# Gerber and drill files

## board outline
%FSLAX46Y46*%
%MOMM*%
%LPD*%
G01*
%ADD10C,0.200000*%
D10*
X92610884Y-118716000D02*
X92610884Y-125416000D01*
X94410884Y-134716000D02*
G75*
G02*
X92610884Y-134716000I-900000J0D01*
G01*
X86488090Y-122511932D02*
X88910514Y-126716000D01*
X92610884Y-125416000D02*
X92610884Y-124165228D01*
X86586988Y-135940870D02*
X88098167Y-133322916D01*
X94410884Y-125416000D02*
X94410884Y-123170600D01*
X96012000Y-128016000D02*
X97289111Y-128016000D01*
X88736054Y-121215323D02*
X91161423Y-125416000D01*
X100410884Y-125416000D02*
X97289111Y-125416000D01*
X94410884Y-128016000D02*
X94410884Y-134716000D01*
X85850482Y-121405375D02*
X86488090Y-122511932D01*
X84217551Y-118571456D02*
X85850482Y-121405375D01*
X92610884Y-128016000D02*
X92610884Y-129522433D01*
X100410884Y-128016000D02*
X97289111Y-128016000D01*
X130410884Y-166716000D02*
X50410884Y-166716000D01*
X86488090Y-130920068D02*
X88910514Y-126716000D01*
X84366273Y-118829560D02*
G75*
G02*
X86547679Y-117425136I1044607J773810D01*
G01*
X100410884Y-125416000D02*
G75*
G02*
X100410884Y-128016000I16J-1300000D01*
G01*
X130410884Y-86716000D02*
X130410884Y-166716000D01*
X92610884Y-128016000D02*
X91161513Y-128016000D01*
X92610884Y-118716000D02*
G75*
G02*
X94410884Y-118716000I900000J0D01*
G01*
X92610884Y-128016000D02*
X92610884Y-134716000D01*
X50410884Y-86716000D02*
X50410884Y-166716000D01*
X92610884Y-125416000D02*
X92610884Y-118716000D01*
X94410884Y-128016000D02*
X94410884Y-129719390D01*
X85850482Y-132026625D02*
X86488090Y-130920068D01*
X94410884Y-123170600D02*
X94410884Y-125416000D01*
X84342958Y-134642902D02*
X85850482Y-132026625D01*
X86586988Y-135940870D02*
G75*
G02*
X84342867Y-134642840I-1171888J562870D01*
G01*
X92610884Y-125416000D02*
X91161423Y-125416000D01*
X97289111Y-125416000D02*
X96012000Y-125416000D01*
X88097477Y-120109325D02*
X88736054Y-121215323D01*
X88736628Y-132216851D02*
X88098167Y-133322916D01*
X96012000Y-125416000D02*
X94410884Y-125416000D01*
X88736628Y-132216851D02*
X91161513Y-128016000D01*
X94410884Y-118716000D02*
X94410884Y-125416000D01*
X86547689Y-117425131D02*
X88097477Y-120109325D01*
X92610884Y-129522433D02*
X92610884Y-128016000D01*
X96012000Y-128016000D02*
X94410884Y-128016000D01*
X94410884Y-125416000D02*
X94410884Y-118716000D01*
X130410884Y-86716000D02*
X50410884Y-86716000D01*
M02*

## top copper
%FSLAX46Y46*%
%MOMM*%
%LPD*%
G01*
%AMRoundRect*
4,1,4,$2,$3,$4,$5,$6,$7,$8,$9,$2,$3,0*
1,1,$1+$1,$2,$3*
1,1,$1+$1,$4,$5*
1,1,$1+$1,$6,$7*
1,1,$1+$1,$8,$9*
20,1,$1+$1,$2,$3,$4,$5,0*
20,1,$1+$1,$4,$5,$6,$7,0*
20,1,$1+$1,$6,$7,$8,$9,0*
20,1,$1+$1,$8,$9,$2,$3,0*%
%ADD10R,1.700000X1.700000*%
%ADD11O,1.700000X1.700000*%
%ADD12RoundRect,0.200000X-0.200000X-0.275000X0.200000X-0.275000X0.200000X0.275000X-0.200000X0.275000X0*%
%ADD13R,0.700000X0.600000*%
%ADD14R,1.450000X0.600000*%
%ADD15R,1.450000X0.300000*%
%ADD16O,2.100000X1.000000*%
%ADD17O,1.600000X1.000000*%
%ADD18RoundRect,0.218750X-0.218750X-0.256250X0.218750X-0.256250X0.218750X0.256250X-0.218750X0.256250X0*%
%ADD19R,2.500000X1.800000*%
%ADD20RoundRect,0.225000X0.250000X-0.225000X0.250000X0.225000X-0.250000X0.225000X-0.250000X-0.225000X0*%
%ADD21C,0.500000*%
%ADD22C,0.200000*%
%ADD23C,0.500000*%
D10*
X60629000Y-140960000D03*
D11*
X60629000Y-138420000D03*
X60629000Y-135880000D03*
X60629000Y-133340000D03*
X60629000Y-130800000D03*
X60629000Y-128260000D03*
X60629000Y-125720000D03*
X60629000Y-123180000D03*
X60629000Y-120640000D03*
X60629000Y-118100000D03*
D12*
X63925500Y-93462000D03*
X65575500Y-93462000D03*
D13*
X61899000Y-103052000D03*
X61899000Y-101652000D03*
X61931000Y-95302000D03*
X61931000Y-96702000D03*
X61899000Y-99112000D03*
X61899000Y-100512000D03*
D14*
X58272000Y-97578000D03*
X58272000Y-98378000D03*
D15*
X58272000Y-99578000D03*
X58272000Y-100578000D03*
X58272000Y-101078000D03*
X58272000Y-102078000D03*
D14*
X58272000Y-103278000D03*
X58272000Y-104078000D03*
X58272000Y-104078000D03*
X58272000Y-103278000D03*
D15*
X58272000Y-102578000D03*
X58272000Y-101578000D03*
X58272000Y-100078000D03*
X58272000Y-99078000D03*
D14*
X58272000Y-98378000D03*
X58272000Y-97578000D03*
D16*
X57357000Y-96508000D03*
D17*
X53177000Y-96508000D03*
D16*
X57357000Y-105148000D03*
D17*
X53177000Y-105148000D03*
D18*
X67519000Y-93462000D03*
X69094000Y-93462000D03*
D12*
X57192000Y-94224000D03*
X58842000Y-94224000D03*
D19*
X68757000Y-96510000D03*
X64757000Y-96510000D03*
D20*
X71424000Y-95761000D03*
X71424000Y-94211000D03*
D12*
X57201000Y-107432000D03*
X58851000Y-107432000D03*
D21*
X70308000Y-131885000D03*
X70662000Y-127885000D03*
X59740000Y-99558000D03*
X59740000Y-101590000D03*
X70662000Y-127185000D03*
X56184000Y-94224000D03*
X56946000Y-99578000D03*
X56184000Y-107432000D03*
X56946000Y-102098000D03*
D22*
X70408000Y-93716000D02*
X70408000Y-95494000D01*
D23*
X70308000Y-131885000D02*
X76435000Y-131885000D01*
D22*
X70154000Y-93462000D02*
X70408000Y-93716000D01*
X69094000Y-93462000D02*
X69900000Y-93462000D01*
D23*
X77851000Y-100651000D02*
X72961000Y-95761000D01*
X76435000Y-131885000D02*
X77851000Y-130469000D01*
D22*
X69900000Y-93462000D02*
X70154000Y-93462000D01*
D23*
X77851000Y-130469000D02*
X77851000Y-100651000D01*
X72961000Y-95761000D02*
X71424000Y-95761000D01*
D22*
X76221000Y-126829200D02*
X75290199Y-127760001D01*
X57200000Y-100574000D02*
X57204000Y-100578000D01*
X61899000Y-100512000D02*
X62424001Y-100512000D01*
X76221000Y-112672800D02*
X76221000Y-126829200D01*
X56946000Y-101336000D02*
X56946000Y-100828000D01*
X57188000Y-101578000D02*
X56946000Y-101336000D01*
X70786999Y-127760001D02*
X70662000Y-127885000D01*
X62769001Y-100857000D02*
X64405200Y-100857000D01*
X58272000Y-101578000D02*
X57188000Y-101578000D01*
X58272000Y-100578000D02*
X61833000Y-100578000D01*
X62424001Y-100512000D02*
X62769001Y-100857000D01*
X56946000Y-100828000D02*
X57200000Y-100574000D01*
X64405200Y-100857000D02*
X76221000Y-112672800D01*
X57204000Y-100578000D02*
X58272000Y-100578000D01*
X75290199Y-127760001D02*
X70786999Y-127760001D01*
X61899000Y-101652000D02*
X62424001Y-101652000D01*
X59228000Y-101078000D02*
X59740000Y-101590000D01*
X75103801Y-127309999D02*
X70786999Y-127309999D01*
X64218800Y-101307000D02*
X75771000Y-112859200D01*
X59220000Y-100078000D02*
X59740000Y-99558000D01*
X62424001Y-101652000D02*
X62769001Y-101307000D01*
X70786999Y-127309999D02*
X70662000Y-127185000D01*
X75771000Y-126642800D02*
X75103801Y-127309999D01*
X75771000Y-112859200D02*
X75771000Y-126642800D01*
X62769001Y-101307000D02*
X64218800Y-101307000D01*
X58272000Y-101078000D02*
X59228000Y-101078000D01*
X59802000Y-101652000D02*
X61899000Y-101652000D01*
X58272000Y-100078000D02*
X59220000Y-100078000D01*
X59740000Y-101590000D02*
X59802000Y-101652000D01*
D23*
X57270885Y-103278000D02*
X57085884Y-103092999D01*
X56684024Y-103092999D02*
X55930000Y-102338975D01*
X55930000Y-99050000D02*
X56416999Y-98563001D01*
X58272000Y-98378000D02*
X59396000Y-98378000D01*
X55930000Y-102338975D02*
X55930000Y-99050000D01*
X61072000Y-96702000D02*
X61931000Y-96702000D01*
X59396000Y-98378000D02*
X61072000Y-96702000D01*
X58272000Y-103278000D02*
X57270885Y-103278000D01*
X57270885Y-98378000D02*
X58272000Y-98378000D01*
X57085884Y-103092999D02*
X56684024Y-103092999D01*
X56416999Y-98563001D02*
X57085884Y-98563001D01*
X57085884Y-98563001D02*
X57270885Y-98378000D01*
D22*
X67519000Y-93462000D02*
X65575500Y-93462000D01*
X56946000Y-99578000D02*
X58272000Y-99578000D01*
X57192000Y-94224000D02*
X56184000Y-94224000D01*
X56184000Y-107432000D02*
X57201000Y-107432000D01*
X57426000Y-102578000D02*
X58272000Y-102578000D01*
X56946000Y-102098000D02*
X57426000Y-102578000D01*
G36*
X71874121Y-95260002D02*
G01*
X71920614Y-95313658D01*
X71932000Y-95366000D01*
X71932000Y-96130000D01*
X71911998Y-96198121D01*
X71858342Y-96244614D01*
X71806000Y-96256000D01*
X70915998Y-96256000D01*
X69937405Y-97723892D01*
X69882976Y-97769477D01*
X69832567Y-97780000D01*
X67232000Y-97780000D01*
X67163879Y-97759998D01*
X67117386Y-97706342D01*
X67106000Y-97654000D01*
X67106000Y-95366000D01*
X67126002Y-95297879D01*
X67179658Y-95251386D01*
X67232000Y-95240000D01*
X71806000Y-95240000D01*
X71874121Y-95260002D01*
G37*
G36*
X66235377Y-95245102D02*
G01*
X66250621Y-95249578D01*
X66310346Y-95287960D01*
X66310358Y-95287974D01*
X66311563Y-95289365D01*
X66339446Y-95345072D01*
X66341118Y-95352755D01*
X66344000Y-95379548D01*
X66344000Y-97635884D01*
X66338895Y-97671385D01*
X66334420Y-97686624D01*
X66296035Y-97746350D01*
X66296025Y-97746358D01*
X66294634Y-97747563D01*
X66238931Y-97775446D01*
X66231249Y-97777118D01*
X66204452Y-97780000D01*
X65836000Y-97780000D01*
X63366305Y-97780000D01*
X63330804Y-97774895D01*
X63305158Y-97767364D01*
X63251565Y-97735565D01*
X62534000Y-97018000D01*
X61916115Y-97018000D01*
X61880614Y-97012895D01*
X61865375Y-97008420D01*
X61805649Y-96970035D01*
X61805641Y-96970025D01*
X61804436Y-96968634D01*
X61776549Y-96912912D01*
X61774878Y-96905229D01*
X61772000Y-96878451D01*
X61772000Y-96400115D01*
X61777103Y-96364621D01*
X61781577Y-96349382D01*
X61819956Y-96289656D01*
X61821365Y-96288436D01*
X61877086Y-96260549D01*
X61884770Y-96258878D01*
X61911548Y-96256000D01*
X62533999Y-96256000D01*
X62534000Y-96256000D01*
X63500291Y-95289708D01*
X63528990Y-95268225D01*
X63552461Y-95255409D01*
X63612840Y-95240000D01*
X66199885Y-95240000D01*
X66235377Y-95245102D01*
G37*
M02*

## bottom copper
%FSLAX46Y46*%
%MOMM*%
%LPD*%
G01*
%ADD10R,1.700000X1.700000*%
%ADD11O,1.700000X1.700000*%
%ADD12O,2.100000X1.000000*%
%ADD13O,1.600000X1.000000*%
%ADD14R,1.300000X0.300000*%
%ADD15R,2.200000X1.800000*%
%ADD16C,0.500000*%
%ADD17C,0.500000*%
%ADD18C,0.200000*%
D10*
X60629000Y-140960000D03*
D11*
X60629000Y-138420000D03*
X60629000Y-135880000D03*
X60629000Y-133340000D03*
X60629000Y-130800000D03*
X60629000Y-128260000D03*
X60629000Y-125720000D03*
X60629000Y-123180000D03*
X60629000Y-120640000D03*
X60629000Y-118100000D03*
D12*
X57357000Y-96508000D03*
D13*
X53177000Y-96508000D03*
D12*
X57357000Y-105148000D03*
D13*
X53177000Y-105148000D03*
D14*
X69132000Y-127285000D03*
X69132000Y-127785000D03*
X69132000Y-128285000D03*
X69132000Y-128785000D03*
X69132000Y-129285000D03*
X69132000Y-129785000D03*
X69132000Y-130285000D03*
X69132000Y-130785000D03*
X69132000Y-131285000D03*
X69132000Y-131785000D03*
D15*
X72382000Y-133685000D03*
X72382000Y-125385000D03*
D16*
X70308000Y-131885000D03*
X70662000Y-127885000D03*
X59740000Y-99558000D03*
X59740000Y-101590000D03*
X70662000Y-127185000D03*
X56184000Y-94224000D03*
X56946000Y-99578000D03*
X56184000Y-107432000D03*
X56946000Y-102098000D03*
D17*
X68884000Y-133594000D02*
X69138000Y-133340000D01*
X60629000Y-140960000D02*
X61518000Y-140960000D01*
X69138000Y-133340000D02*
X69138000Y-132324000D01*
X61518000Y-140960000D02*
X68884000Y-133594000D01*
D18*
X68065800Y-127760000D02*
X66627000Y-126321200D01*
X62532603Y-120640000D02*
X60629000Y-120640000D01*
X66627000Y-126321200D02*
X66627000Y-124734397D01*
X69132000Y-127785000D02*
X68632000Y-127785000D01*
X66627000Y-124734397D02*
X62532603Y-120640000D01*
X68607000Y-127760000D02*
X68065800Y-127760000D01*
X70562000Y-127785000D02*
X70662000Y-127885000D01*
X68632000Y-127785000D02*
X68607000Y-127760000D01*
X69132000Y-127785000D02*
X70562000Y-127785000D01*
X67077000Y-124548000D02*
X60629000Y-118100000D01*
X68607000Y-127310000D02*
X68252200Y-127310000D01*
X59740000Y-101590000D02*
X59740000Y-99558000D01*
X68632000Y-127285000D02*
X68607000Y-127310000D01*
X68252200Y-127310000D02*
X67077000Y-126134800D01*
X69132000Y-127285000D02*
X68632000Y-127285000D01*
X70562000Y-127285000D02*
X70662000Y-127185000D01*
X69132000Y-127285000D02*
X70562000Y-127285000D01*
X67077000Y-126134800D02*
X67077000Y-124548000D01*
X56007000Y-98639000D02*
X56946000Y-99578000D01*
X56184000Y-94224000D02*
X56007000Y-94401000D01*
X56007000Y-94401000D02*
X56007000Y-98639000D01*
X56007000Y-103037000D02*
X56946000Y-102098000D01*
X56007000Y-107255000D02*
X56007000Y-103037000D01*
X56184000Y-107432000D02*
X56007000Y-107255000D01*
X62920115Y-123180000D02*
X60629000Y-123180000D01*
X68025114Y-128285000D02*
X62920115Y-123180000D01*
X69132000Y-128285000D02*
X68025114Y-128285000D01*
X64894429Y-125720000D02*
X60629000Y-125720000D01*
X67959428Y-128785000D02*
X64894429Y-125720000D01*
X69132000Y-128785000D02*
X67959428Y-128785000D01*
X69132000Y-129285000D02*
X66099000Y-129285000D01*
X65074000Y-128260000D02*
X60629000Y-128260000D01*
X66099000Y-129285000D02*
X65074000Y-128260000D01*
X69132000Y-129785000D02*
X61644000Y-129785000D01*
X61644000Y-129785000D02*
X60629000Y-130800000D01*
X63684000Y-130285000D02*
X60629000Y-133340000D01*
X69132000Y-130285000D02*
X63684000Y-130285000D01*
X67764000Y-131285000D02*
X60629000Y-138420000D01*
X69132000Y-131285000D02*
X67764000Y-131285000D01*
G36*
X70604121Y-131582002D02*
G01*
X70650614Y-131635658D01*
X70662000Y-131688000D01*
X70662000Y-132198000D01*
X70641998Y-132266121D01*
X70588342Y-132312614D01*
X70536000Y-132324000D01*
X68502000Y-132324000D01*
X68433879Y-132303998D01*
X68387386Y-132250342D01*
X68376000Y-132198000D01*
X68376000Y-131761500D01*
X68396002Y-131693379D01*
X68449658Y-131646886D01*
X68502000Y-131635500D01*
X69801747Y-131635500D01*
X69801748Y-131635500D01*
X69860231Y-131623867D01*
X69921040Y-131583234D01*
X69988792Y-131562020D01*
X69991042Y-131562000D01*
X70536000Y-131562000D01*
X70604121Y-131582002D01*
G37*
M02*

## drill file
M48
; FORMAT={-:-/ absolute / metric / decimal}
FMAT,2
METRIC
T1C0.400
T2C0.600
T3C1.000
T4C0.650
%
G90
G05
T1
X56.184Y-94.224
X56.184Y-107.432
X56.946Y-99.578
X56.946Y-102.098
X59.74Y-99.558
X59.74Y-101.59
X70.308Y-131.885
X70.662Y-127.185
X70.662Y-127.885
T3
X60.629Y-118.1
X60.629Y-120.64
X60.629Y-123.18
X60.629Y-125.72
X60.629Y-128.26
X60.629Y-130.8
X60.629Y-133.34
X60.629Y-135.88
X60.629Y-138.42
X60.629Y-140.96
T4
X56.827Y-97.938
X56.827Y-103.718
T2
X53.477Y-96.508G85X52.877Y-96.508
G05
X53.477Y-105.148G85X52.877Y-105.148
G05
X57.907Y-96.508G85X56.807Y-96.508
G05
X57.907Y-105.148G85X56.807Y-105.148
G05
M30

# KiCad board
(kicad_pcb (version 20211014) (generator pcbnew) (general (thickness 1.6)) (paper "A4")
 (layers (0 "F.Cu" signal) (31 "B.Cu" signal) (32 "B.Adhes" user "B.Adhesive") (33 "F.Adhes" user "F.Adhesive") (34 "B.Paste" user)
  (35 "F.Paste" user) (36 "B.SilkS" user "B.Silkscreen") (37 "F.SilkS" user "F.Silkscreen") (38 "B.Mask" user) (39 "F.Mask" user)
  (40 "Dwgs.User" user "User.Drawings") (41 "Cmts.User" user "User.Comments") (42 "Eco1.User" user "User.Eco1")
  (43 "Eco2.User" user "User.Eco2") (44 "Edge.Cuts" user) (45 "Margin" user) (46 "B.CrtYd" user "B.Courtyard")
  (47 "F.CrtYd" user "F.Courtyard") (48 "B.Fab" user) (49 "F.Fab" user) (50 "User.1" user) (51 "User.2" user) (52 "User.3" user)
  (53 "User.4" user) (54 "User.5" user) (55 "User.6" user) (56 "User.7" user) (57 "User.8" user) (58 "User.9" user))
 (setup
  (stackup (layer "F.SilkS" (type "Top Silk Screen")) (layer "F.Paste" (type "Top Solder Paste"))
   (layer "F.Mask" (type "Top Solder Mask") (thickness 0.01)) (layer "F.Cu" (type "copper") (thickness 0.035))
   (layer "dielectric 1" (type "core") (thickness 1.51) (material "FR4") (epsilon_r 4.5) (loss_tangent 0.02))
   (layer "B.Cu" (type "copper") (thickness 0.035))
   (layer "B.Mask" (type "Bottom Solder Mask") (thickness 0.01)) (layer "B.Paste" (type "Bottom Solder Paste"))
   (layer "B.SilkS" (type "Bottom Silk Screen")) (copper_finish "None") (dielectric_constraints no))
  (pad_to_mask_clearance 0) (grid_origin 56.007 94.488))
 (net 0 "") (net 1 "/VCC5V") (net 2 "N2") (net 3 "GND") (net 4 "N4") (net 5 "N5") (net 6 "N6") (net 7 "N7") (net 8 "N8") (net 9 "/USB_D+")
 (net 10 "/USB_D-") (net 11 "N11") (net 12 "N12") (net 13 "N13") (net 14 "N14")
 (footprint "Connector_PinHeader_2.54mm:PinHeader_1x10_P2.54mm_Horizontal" (layer "F.Cu") (at 60.629 140.96 180)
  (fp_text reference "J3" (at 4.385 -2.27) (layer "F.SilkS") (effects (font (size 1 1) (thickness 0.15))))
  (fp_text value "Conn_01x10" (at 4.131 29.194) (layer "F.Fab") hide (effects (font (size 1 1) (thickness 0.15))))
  (pad "1" thru_hole rect (at 0 0 180) (size 1.7 1.7) (drill 1) (layers *.Cu *.Mask) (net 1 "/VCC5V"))
  (pad "2" thru_hole oval (at 0 2.54 180) (size 1.7 1.7) (drill 1) (layers *.Cu *.Mask) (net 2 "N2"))
  (pad "3" thru_hole oval (at 0 5.08 180) (size 1.7 1.7) (drill 1) (layers *.Cu *.Mask) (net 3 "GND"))
  (pad "4" thru_hole oval (at 0 7.62 180) (size 1.7 1.7) (drill 1) (layers *.Cu *.Mask) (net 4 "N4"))
  (pad "5" thru_hole oval (at 0 10.16 180) (size 1.7 1.7) (drill 1) (layers *.Cu *.Mask) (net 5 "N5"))
  (pad "6" thru_hole oval (at 0 12.7 180) (size 1.7 1.7) (drill 1) (layers *.Cu *.Mask) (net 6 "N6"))
  (pad "7" thru_hole oval (at 0 15.24 180) (size 1.7 1.7) (drill 1) (layers *.Cu *.Mask) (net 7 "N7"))
  (pad "8" thru_hole oval (at 0 17.78 180) (size 1.7 1.7) (drill 1) (layers *.Cu *.Mask) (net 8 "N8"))
  (pad "9" thru_hole oval (at 0 20.32 180) (size 1.7 1.7) (drill 1) (layers *.Cu *.Mask) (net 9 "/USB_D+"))
  (pad "10" thru_hole oval (at 0 22.86 180) (size 1.7 1.7) (drill 1) (layers *.Cu *.Mask) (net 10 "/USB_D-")))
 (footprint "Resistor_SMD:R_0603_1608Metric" (layer "F.Cu") (at 64.7505 93.462)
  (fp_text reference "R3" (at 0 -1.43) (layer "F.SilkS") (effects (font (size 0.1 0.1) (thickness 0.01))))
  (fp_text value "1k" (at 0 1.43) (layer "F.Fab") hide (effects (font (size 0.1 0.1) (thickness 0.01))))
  (pad "1" smd roundrect (at -0.825 0) (size 0.8 0.95) (layers "F.Cu" "F.Paste" "F.Mask") (roundrect_rratio 0.25) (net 3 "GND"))
  (pad "2" smd roundrect (at 0.825 0) (size 0.8 0.95) (layers "F.Cu" "F.Paste" "F.Mask") (roundrect_rratio 0.25) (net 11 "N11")))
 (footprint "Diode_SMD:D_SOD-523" (layer "F.Cu") (at 61.899 102.352 90)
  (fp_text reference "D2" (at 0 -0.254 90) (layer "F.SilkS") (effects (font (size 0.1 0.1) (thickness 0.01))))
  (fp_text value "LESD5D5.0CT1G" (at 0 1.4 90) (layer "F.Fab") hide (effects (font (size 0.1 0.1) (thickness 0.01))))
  (pad "1" smd rect (at -0.7 0 270) (size 0.6 0.7) (layers "F.Cu" "F.Paste" "F.Mask") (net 3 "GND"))
  (pad "2" smd rect (at 0.7 0 270) (size 0.6 0.7) (layers "F.Cu" "F.Paste" "F.Mask") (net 10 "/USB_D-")))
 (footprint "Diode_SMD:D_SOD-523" (layer "F.Cu") (at 61.931 96.002 -90)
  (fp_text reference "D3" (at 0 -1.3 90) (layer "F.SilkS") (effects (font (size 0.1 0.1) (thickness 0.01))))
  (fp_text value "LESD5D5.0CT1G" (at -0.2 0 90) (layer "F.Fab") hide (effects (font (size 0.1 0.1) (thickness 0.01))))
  (pad "1" smd rect (at -0.7 0 90) (size 0.6 0.7) (layers "F.Cu" "F.Paste" "F.Mask") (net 3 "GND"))
  (pad "2" smd rect (at 0.7 0 90) (size 0.6 0.7) (layers "F.Cu" "F.Paste" "F.Mask") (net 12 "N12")))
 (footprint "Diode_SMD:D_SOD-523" (layer "F.Cu") (at 61.899 99.812 -90)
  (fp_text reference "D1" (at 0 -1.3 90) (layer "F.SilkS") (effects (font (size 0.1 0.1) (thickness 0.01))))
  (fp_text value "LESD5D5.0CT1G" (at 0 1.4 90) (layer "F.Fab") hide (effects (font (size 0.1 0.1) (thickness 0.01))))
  (pad "1" smd rect (at -0.7 0 90) (size 0.6 0.7) (layers "F.Cu" "F.Paste" "F.Mask") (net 3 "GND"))
  (pad "2" smd rect (at 0.7 0 90) (size 0.6 0.7) (layers "F.Cu" "F.Paste" "F.Mask") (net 9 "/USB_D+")))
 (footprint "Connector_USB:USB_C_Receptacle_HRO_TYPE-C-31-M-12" (layer "F.Cu") (at 54.227 100.828 -90)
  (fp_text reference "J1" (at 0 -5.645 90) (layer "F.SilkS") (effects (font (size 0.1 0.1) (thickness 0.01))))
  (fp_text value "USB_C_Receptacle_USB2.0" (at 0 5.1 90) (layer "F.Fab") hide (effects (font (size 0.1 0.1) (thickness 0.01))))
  (pad "" np_thru_hole circle (at 2.89 -2.6 270) (size 0.65 0.65) (drill 0.65) (layers *.Cu *.Mask))
  (pad "" np_thru_hole circle (at -2.89 -2.6 270) (size 0.65 0.65) (drill 0.65) (layers *.Cu *.Mask))
  (pad "A1" smd rect (at -3.25 -4.045 270) (size 0.6 1.45) (layers "F.Cu" "F.Paste" "F.Mask") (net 3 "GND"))
  (pad "A4" smd rect (at -2.45 -4.045 270) (size 0.6 1.45) (layers "F.Cu" "F.Paste" "F.Mask") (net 12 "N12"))
  (pad "A5" smd rect (at -1.25 -4.045 270) (size 0.3 1.45) (layers "F.Cu" "F.Paste" "F.Mask") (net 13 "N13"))
  (pad "A6" smd rect locked (at -0.25 -4.045 270) (size 0.3 1.45) (layers "F.Cu" "F.Paste" "F.Mask") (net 9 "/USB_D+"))
  (pad "A7" smd rect (at 0.25 -4.045 270) (size 0.3 1.45) (layers "F.Cu" "F.Paste" "F.Mask") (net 10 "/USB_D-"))
  (pad "A8" smd rect (at 1.25 -4.045 270) (size 0.3 1.45) (layers "F.Cu" "F.Paste" "F.Mask") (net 3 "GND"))
  (pad "A9" smd rect (at 2.45 -4.045 270) (size 0.6 1.45) (layers "F.Cu" "F.Paste" "F.Mask") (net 12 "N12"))
  (pad "A12" smd rect (at 3.25 -4.045 270) (size 0.6 1.45) (layers "F.Cu" "F.Paste" "F.Mask") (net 3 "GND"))
  (pad "B1" smd rect (at 3.25 -4.045 270) (size 0.6 1.45) (layers "F.Cu" "F.Paste" "F.Mask") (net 3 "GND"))
  (pad "B4" smd rect (at 2.45 -4.045 270) (size 0.6 1.45) (layers "F.Cu" "F.Paste" "F.Mask") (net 12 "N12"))
  (pad "B5" smd rect (at 1.75 -4.045 270) (size 0.3 1.45) (layers "F.Cu" "F.Paste" "F.Mask") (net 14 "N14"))
  (pad "B6" smd rect (at 0.75 -4.045 270) (size 0.3 1.45) (layers "F.Cu" "F.Paste" "F.Mask") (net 9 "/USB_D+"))
  (pad "B7" smd rect (at -0.75 -4.045 270) (size 0.3 1.45) (layers "F.Cu" "F.Paste" "F.Mask") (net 10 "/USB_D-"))
  (pad "B8" smd rect (at -1.75 -4.045 270) (size 0.3 1.45) (layers "F.Cu" "F.Paste" "F.Mask") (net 3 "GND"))
  (pad "B9" smd rect (at -2.45 -4.045 270) (size 0.6 1.45) (layers "F.Cu" "F.Paste" "F.Mask") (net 12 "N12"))
  (pad "B12" smd rect (at -3.25 -4.045 270) (size 0.6 1.45) (layers "F.Cu" "F.Paste" "F.Mask") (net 3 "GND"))
  (pad "S1" thru_hole oval (at -4.32 -3.13 270) (size 1 2.1) (drill oval 0.6 1.7) (layers *.Cu *.Mask) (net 3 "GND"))
  (pad "S1" thru_hole oval (at -4.32 1.05 270) (size 1 1.6) (drill oval 0.6 1.2) (layers *.Cu *.Mask) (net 3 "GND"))
  (pad "S1" thru_hole oval (at 4.32 -3.13 270) (size 1 2.1) (drill oval 0.6 1.7) (layers *.Cu *.Mask) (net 3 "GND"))
  (pad "S1" thru_hole oval (at 4.32 1.05 270) (size 1 1.6) (drill oval 0.6 1.2) (layers *.Cu *.Mask) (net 3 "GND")))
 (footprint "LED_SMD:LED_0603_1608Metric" (layer "F.Cu") (at 68.3065 93.462)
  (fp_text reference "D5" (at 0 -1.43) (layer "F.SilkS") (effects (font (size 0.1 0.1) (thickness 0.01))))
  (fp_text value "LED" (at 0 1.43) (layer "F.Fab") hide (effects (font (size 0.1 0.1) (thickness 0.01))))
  (pad "1" smd roundrect (at -0.7875 0) (size 0.875 0.95) (layers "F.Cu" "F.Paste" "F.Mask") (roundrect_rratio 0.25) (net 11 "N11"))
  (pad "2" smd roundrect (at 0.7875 0) (size 0.875 0.95) (layers "F.Cu" "F.Paste" "F.Mask") (roundrect_rratio 0.25) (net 1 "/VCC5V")))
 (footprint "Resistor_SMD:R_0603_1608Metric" (layer "F.Cu") (at 58.017 94.224)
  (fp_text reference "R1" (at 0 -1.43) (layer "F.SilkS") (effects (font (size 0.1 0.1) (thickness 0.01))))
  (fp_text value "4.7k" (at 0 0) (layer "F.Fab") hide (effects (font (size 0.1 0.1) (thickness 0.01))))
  (pad "1" smd roundrect (at -0.825 0) (size 0.8 0.95) (layers "F.Cu" "F.Paste" "F.Mask") (roundrect_rratio 0.25) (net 13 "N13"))
  (pad "2" smd roundrect (at 0.825 0) (size 0.8 0.95) (layers "F.Cu" "F.Paste" "F.Mask") (roundrect_rratio 0.25) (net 3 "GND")))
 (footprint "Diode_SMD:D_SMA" (layer "F.Cu") (at 66.757 96.51 180)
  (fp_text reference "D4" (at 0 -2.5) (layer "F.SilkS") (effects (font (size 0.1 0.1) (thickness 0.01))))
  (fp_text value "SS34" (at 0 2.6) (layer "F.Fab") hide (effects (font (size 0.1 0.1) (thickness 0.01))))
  (pad "1" smd rect (at -2 0 180) (size 2.5 1.8) (layers "F.Cu" "F.Paste" "F.Mask") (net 1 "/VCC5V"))
  (pad "2" smd rect (at 2 0 180) (size 2.5 1.8) (layers "F.Cu" "F.Paste" "F.Mask") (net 12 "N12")))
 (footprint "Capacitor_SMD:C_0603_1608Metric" (layer "F.Cu") (at 71.424 94.986 90)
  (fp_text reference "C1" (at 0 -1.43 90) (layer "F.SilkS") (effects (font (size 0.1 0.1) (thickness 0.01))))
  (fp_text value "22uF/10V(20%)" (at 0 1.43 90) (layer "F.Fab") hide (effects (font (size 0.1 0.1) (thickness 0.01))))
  (pad "1" smd roundrect (at -0.775 0 90) (size 0.9 0.95) (layers "F.Cu" "F.Paste" "F.Mask") (roundrect_rratio 0.25) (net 1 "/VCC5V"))
  (pad "2" smd roundrect (at 0.775 0 90) (size 0.9 0.95) (layers "F.Cu" "F.Paste" "F.Mask") (roundrect_rratio 0.25) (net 3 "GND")))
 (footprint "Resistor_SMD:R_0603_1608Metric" (layer "F.Cu") (at 58.026 107.432)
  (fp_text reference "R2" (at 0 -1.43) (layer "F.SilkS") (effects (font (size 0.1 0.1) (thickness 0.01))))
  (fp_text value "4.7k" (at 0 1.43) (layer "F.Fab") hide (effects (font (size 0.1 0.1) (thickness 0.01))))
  (pad "1" smd roundrect (at -0.825 0) (size 0.8 0.95) (layers "F.Cu" "F.Paste" "F.Mask") (roundrect_rratio 0.25) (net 14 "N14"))
  (pad "2" smd roundrect (at 0.825 0) (size 0.8 0.95) (layers "F.Cu" "F.Paste" "F.Mask") (roundrect_rratio 0.25) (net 3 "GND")))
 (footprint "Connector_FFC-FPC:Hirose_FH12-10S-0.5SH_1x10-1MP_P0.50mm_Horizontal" (layer "B.Cu") (at 70.982 129.535 -90)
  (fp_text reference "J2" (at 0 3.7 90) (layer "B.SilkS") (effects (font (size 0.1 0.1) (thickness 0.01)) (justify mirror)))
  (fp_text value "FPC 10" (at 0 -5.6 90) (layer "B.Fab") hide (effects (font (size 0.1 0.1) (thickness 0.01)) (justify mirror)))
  (pad "1" smd rect (at -2.25 1.85 270) (size 0.3 1.3) (layers "B.Cu" "B.Paste" "B.Mask") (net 10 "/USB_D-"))
  (pad "2" smd rect (at -1.75 1.85 270) (size 0.3 1.3) (layers "B.Cu" "B.Paste" "B.Mask") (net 9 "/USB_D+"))
  (pad "3" smd rect (at -1.25 1.85 270) (size 0.3 1.3) (layers "B.Cu" "B.Paste" "B.Mask") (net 8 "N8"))
  (pad "4" smd rect (at -0.75 1.85 270) (size 0.3 1.3) (layers "B.Cu" "B.Paste" "B.Mask") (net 7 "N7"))
  (pad "5" smd rect (at -0.25 1.85 270) (size 0.3 1.3) (layers "B.Cu" "B.Paste" "B.Mask") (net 6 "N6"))
  (pad "6" smd rect (at 0.25 1.85 270) (size 0.3 1.3) (layers "B.Cu" "B.Paste" "B.Mask") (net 5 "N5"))
  (pad "7" smd rect (at 0.75 1.85 270) (size 0.3 1.3) (layers "B.Cu" "B.Paste" "B.Mask") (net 4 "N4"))
  (pad "8" smd rect (at 1.25 1.85 270) (size 0.3 1.3) (layers "B.Cu" "B.Paste" "B.Mask") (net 3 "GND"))
  (pad "9" smd rect (at 1.75 1.85 270) (size 0.3 1.3) (layers "B.Cu" "B.Paste" "B.Mask") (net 2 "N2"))
  (pad "10" smd rect (at 2.25 1.85 270) (size 0.3 1.3) (layers "B.Cu" "B.Paste" "B.Mask") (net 1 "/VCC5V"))
  (pad "MP" smd rect (at 4.15 -1.4 270) (size 1.8 2.2) (layers "B.Cu" "B.Paste" "B.Mask"))
  (pad "MP" smd rect (at -4.15 -1.4 270) (size 1.8 2.2) (layers "B.Cu" "B.Paste" "B.Mask")))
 (gr_line (start 92.610884 118.716) (end 92.610884 125.416) (layer "Edge.Cuts") (width 0.2))
 (gr_arc (start 94.410884 134.716) (mid 93.510884 135.616) (end 92.610884 134.716) (layer "Edge.Cuts") (width 0.2))
 (gr_line (start 86.48809 122.511932) (end 88.910514 126.716) (layer "Edge.Cuts") (width 0.2))
 (gr_line (start 92.610884 125.416) (end 92.610884 124.165228) (layer "Edge.Cuts") (width 0.2))
 (gr_line (start 86.586988 135.94087) (end 88.098167 133.322916) (layer "Edge.Cuts") (width 0.2))
 (gr_line (start 94.410884 125.416) (end 94.410884 123.1706) (layer "Edge.Cuts") (width 0.2))
 (gr_line (start 96.012 128.016) (end 97.289111 128.016) (layer "Edge.Cuts") (width 0.2))
 (gr_line (start 88.736054 121.215323) (end 91.161423 125.416) (layer "Edge.Cuts") (width 0.2))
 (gr_line (start 100.410884 125.416) (end 97.289111 125.416) (layer "Edge.Cuts") (width 0.2))
 (gr_line (start 94.410884 128.016) (end 94.410884 134.716) (layer "Edge.Cuts") (width 0.2))
 (gr_line (start 85.850482 121.405375) (end 86.48809 122.511932) (layer "Edge.Cuts") (width 0.2))
 (gr_line (start 84.217551 118.571456) (end 85.850482 121.405375) (layer "Edge.Cuts") (width 0.2))
 (gr_line (start 92.610884 128.016) (end 92.610884 129.522433) (layer "Edge.Cuts") (width 0.2))
 (gr_line (start 100.410884 128.016) (end 97.289111 128.016) (layer "Edge.Cuts") (width 0.2))
 (gr_line (start 130.410884 166.716) (end 50.410884 166.716) (layer "Edge.Cuts") (width 0.2))
 (gr_line (start 86.48809 130.920068) (end 88.910514 126.716) (layer "Edge.Cuts") (width 0.2))
 (gr_arc (start 84.366273 118.82956) (mid 84.707158 116.962691) (end 86.547689 117.425131) (layer "Edge.Cuts") (width 0.2))
 (gr_arc (start 100.410884 125.416) (mid 101.710884 126.716) (end 100.410884 128.016) (layer "Edge.Cuts") (width 0.2))
 (gr_line (start 130.410884 86.716) (end 130.410884 166.716) (layer "Edge.Cuts") (width 0.2))
 (gr_line (start 92.610884 128.016) (end 91.161513 128.016) (layer "Edge.Cuts") (width 0.2))
 (gr_arc (start 92.610884 118.716) (mid 93.510884 117.816) (end 94.410884 118.716) (layer "Edge.Cuts") (width 0.2))
 (gr_line (start 92.610884 128.016) (end 92.610884 134.716) (layer "Edge.Cuts") (width 0.2))
 (gr_line (start 50.410884 86.716) (end 50.410884 166.716) (layer "Edge.Cuts") (width 0.2))
 (gr_line (start 92.610884 125.416) (end 92.610884 118.716) (layer "Edge.Cuts") (width 0.2))
 (gr_line (start 94.410884 128.016) (end 94.410884 129.71939) (layer "Edge.Cuts") (width 0.2))
 (gr_line (start 85.850482 132.026625) (end 86.48809 130.920068) (layer "Edge.Cuts") (width 0.2))
 (gr_line (start 94.410884 123.1706) (end 94.410884 125.416) (layer "Edge.Cuts") (width 0.2))
 (gr_line (start 84.342958 134.642902) (end 85.850482 132.026625) (layer "Edge.Cuts") (width 0.2))
 (gr_arc (start 86.586988 135.94087) (mid 84.764255 136.503343) (end 84.342958 134.642902) (layer "Edge.Cuts") (width 0.2))
 (gr_line (start 92.610884 125.416) (end 91.161423 125.416) (layer "Edge.Cuts") (width 0.2))
 (gr_line (start 97.289111 125.416) (end 96.012 125.416) (layer "Edge.Cuts") (width 0.2))
 (gr_line (start 88.097477 120.109325) (end 88.736054 121.215323) (layer "Edge.Cuts") (width 0.2))
 (gr_line (start 88.736628 132.216851) (end 88.098167 133.322916) (layer "Edge.Cuts") (width 0.2))
 (gr_line (start 96.012 125.416) (end 94.410884 125.416) (layer "Edge.Cuts") (width 0.2))
 (gr_line (start 88.736628 132.216851) (end 91.161513 128.016) (layer "Edge.Cuts") (width 0.2))
 (gr_line (start 94.410884 118.716) (end 94.410884 125.416) (layer "Edge.Cuts") (width 0.2))
 (gr_line (start 86.547689 117.425131) (end 88.097477 120.109325) (layer "Edge.Cuts") (width 0.2))
 (gr_line (start 92.610884 129.522433) (end 92.610884 128.016) (layer "Edge.Cuts") (width 0.2))
 (gr_line (start 96.012 128.016) (end 94.410884 128.016) (layer "Edge.Cuts") (width 0.2))
 (gr_line (start 94.410884 125.416) (end 94.410884 118.716) (layer "Edge.Cuts") (width 0.2))
 (gr_line (start 130.410884 86.716) (end 50.410884 86.716) (layer "Edge.Cuts") (width 0.2))
 (segment (start 70.408 93.716) (end 70.408 95.494) (width 0.2) (layer "F.Cu") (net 1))
 (segment (start 70.308 131.885) (end 76.435 131.885) (width 0.5) (layer "F.Cu") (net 1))
 (segment (start 70.154 93.462) (end 70.408 93.716) (width 0.2) (layer "F.Cu") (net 1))
 (segment (start 69.094 93.462) (end 69.9 93.462) (width 0.2) (layer "F.Cu") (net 1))
 (segment (start 77.851 100.651) (end 72.961 95.761) (width 0.5) (layer "F.Cu") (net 1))
 (segment (start 76.435 131.885) (end 77.851 130.469) (width 0.5) (layer "F.Cu") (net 1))
 (segment (start 69.9 93.462) (end 70.154 93.462) (width 0.2) (layer "F.Cu") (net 1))
 (segment (start 77.851 130.469) (end 77.851 100.651) (width 0.5) (layer "F.Cu") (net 1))
 (segment (start 72.961 95.761) (end 71.424 95.761) (width 0.5) (layer "F.Cu") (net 1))
 (via (at 70.308 131.885) (size 0.5) (drill 0.4) (layers "F.Cu" "B.Cu") (free) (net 1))
 (segment (start 68.884 133.594) (end 69.138 133.34) (width 0.5) (layer "B.Cu") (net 1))
 (segment (start 60.629 140.96) (end 61.518 140.96) (width 0.5) (layer "B.Cu") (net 1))
 (segment (start 69.138 133.34) (end 69.138 132.324) (width 0.5) (layer "B.Cu") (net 1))
 (segment (start 61.518 140.96) (end 68.884 133.594) (width 0.5) (layer "B.Cu") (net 1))
 (segment (start 76.221 126.8292) (end 75.290199 127.760001) (width 0.2) (layer "F.Cu") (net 9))
 (segment (start 57.2 100.574) (end 57.204 100.578) (width 0.2) (layer "F.Cu") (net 9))
 (segment (start 61.899 100.512) (end 62.424001 100.512) (width 0.2) (layer "F.Cu") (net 9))
 (segment (start 76.221 112.6728) (end 76.221 126.8292) (width 0.2) (layer "F.Cu") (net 9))
 (segment (start 56.946 101.336) (end 56.946 100.828) (width 0.2) (layer "F.Cu") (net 9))
 (segment (start 57.188 101.578) (end 56.946 101.336) (width 0.2) (layer "F.Cu") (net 9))
 (segment (start 70.786999 127.760001) (end 70.662 127.885) (width 0.2) (layer "F.Cu") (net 9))
 (segment (start 62.769001 100.857) (end 64.4052 100.857) (width 0.2) (layer "F.Cu") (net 9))
 (segment (start 58.272 101.578) (end 57.188 101.578) (width 0.2) (layer "F.Cu") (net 9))
 (segment (start 58.272 100.578) (end 61.833 100.578) (width 0.2) (layer "F.Cu") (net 9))
 (segment (start 62.424001 100.512) (end 62.769001 100.857) (width 0.2) (layer "F.Cu") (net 9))
 (segment (start 56.946 100.828) (end 57.2 100.574) (width 0.2) (layer "F.Cu") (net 9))
 (segment (start 64.4052 100.857) (end 76.221 112.6728) (width 0.2) (layer "F.Cu") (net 9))
 (segment (start 57.204 100.578) (end 58.272 100.578) (width 0.2) (layer "F.Cu") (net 9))
 (segment (start 75.290199 127.760001) (end 70.786999 127.760001) (width 0.2) (layer "F.Cu") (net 9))
 (via (at 70.662 127.885) (size 0.5) (drill 0.4) (layers "F.Cu" "B.Cu") (free) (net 9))
 (segment (start 68.0658 127.76) (end 66.627 126.3212) (width 0.2) (layer "B.Cu") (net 9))
 (segment (start 62.532603 120.64) (end 60.629 120.64) (width 0.2) (layer "B.Cu") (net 9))
 (segment (start 66.627 126.3212) (end 66.627 124.734397) (width 0.2) (layer "B.Cu") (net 9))
 (segment (start 69.132 127.785) (end 68.632 127.785) (width 0.2) (layer "B.Cu") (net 9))
 (segment (start 66.627 124.734397) (end 62.532603 120.64) (width 0.2) (layer "B.Cu") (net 9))
 (segment (start 68.607 127.76) (end 68.0658 127.76) (width 0.2) (layer "B.Cu") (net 9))
 (segment (start 70.562 127.785) (end 70.662 127.885) (width 0.2) (layer "B.Cu") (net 9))
 (segment (start 68.632 127.785) (end 68.607 127.76) (width 0.2) (layer "B.Cu") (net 9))
 (segment (start 69.132 127.785) (end 70.562 127.785) (width 0.2) (layer "B.Cu") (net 9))
 (segment (start 61.899 101.652) (end 62.424001 101.652) (width 0.2) (layer "F.Cu") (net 10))
 (segment (start 59.228 101.078) (end 59.74 101.59) (width 0.2) (layer "F.Cu") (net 10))
 (segment (start 75.103801 127.309999) (end 70.786999 127.309999) (width 0.2) (layer "F.Cu") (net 10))
 (segment (start 64.2188 101.307) (end 75.771 112.8592) (width 0.2) (layer "F.Cu") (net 10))
 (segment (start 59.22 100.078) (end 59.74 99.558) (width 0.2) (layer "F.Cu") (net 10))
 (segment (start 62.424001 101.652) (end 62.769001 101.307) (width 0.2) (layer "F.Cu") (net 10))
 (segment (start 70.786999 127.309999) (end 70.662 127.185) (width 0.2) (layer "F.Cu") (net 10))
 (segment (start 75.771 126.6428) (end 75.103801 127.309999) (width 0.2) (layer "F.Cu") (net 10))
 (segment (start 75.771 112.8592) (end 75.771 126.6428) (width 0.2) (layer "F.Cu") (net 10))
 (segment (start 62.769001 101.307) (end 64.2188 101.307) (width 0.2) (layer "F.Cu") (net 10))
 (segment (start 58.272 101.078) (end 59.228 101.078) (width 0.2) (layer "F.Cu") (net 10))
 (segment (start 59.802 101.652) (end 61.899 101.652) (width 0.2) (layer "F.Cu") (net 10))
 (segment (start 58.272 100.078) (end 59.22 100.078) (width 0.2) (layer "F.Cu") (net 10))
 (segment (start 59.74 101.59) (end 59.802 101.652) (width 0.2) (layer "F.Cu") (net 10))
 (via (at 59.74 99.558) (size 0.5) (drill 0.4) (layers "F.Cu" "B.Cu") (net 10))
 (via (at 59.74 101.59) (size 0.5) (drill 0.4) (layers "F.Cu" "B.Cu") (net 10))
 (via (at 70.662 127.185) (size 0.5) (drill 0.4) (layers "F.Cu" "B.Cu") (free) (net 10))
 (segment (start 67.077 124.548) (end 60.629 118.1) (width 0.2) (layer "B.Cu") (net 10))
 (segment (start 68.607 127.31) (end 68.2522 127.31) (width 0.2) (layer "B.Cu") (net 10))
 (segment (start 59.74 101.59) (end 59.74 99.558) (width 0.2) (layer "B.Cu") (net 10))
 (segment (start 68.632 127.285) (end 68.607 127.31) (width 0.2) (layer "B.Cu") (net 10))
 (segment (start 68.2522 127.31) (end 67.077 126.1348) (width 0.2) (layer "B.Cu") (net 10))
 (segment (start 69.132 127.285) (end 68.632 127.285) (width 0.2) (layer "B.Cu") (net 10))
 (segment (start 70.562 127.285) (end 70.662 127.185) (width 0.2) (layer "B.Cu") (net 10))
 (segment (start 69.132 127.285) (end 70.562 127.285) (width 0.2) (layer "B.Cu") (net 10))
 (segment (start 67.077 126.1348) (end 67.077 124.548) (width 0.2) (layer "B.Cu") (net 10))
 (segment (start 57.270885 103.278) (end 57.085884 103.092999) (width 0.5) (layer "F.Cu") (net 12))
 (segment (start 56.684024 103.092999) (end 55.93 102.338975) (width 0.5) (layer "F.Cu") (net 12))
 (segment (start 55.93 99.05) (end 56.416999 98.563001) (width 0.5) (layer "F.Cu") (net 12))
 (segment (start 58.272 98.378) (end 59.396 98.378) (width 0.5) (layer "F.Cu") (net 12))
 (segment (start 55.93 102.338975) (end 55.93 99.05) (width 0.5) (layer "F.Cu") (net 12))
 (segment (start 61.072 96.702) (end 61.931 96.702) (width 0.5) (layer "F.Cu") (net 12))
 (segment (start 59.396 98.378) (end 61.072 96.702) (width 0.5) (layer "F.Cu") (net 12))
 (segment (start 58.272 103.278) (end 57.270885 103.278) (width 0.5) (layer "F.Cu") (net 12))
 (segment (start 57.270885 98.378) (end 58.272 98.378) (width 0.5) (layer "F.Cu") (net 12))
 (segment (start 57.085884 103.092999) (end 56.684024 103.092999) (width 0.5) (layer "F.Cu") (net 12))
 (segment (start 56.416999 98.563001) (end 57.085884 98.563001) (width 0.5) (layer "F.Cu") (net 12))
 (segment (start 57.085884 98.563001) (end 57.270885 98.378) (width 0.5) (layer "F.Cu") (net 12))
 (segment (start 67.519 93.462) (end 65.5755 93.462) (width 0.2) (layer "F.Cu") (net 11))
 (segment (start 56.946 99.578) (end 58.272 99.578) (width 0.2) (layer "F.Cu") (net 13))
 (segment (start 57.192 94.224) (end 56.184 94.224) (width 0.2) (layer "F.Cu") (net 13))
 (via (at 56.184 94.224) (size 0.5) (drill 0.4) (layers "F.Cu" "B.Cu") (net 13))
 (via (at 56.946 99.578) (size 0.5) (drill 0.4) (layers "F.Cu" "B.Cu") (free) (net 13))
 (segment (start 56.007 98.639) (end 56.946 99.578) (width 0.2) (layer "B.Cu") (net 13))
 (segment (start 56.184 94.224) (end 56.007 94.401) (width 0.2) (layer "B.Cu") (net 13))
 (segment (start 56.007 94.401) (end 56.007 98.639) (width 0.2) (layer "B.Cu") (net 13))
 (segment (start 56.184 107.432) (end 57.201 107.432) (width 0.2) (layer "F.Cu") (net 14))
 (segment (start 57.426 102.578) (end 58.272 102.578) (width 0.2) (layer "F.Cu") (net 14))
 (segment (start 56.946 102.098) (end 57.426 102.578) (width 0.2) (layer "F.Cu") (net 14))
 (via (at 56.184 107.432) (size 0.5) (drill 0.4) (layers "F.Cu" "B.Cu") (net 14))
 (via (at 56.946 102.098) (size 0.5) (drill 0.4) (layers "F.Cu" "B.Cu") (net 14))
 (segment (start 56.007 103.037) (end 56.946 102.098) (width 0.2) (layer "B.Cu") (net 14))
 (segment (start 56.007 107.255) (end 56.007 103.037) (width 0.2) (layer "B.Cu") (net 14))
 (segment (start 56.184 107.432) (end 56.007 107.255) (width 0.2) (layer "B.Cu") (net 14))
 (segment (start 62.920115 123.18) (end 60.629 123.18) (width 0.2) (layer "B.Cu") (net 8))
 (segment (start 68.025114 128.285) (end 62.920115 123.18) (width 0.2) (layer "B.Cu") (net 8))
 (segment (start 69.132 128.285) (end 68.025114 128.285) (width 0.2) (layer "B.Cu") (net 8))
 (segment (start 64.894429 125.72) (end 60.629 125.72) (width 0.2) (layer "B.Cu") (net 7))
 (segment (start 67.959428 128.785) (end 64.894429 125.72) (width 0.2) (layer "B.Cu") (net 7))
 (segment (start 69.132 128.785) (end 67.959428 128.785) (width 0.2) (layer "B.Cu") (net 7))
 (segment (start 69.132 129.285) (end 66.099 129.285) (width 0.2) (layer "B.Cu") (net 6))
 (segment (start 65.074 128.26) (end 60.629 128.26) (width 0.2) (layer "B.Cu") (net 6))
 (segment (start 66.099 129.285) (end 65.074 128.26) (width 0.2) (layer "B.Cu") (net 6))
 (segment (start 69.132 129.785) (end 61.644 129.785) (width 0.2) (layer "B.Cu") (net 5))
 (segment (start 61.644 129.785) (end 60.629 130.8) (width 0.2) (layer "B.Cu") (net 5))
 (segment (start 63.684 130.285) (end 60.629 133.34) (width 0.2) (layer "B.Cu") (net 4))
 (segment (start 69.132 130.285) (end 63.684 130.285) (width 0.2) (layer "B.Cu") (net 4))
 (segment (start 67.764 131.285) (end 60.629 138.42) (width 0.2) (layer "B.Cu") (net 2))
 (segment (start 69.132 131.285) (end 67.764 131.285) (width 0.2) (layer "B.Cu") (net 2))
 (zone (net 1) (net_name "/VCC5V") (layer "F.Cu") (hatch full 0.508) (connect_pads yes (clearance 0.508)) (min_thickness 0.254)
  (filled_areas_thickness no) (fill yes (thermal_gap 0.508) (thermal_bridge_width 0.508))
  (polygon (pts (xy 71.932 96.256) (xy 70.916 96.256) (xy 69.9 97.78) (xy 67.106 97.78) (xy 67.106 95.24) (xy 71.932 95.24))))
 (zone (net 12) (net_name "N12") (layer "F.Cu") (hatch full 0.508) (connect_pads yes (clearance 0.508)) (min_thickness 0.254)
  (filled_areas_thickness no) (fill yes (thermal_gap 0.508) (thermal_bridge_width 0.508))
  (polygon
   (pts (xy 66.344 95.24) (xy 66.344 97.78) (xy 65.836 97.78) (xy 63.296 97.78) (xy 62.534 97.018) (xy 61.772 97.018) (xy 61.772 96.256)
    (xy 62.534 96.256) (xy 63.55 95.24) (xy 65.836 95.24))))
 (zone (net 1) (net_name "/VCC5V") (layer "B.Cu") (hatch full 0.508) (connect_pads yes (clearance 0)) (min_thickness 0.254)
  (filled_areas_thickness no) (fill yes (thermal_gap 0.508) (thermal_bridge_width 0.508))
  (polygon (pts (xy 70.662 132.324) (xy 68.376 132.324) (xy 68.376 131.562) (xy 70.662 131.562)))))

